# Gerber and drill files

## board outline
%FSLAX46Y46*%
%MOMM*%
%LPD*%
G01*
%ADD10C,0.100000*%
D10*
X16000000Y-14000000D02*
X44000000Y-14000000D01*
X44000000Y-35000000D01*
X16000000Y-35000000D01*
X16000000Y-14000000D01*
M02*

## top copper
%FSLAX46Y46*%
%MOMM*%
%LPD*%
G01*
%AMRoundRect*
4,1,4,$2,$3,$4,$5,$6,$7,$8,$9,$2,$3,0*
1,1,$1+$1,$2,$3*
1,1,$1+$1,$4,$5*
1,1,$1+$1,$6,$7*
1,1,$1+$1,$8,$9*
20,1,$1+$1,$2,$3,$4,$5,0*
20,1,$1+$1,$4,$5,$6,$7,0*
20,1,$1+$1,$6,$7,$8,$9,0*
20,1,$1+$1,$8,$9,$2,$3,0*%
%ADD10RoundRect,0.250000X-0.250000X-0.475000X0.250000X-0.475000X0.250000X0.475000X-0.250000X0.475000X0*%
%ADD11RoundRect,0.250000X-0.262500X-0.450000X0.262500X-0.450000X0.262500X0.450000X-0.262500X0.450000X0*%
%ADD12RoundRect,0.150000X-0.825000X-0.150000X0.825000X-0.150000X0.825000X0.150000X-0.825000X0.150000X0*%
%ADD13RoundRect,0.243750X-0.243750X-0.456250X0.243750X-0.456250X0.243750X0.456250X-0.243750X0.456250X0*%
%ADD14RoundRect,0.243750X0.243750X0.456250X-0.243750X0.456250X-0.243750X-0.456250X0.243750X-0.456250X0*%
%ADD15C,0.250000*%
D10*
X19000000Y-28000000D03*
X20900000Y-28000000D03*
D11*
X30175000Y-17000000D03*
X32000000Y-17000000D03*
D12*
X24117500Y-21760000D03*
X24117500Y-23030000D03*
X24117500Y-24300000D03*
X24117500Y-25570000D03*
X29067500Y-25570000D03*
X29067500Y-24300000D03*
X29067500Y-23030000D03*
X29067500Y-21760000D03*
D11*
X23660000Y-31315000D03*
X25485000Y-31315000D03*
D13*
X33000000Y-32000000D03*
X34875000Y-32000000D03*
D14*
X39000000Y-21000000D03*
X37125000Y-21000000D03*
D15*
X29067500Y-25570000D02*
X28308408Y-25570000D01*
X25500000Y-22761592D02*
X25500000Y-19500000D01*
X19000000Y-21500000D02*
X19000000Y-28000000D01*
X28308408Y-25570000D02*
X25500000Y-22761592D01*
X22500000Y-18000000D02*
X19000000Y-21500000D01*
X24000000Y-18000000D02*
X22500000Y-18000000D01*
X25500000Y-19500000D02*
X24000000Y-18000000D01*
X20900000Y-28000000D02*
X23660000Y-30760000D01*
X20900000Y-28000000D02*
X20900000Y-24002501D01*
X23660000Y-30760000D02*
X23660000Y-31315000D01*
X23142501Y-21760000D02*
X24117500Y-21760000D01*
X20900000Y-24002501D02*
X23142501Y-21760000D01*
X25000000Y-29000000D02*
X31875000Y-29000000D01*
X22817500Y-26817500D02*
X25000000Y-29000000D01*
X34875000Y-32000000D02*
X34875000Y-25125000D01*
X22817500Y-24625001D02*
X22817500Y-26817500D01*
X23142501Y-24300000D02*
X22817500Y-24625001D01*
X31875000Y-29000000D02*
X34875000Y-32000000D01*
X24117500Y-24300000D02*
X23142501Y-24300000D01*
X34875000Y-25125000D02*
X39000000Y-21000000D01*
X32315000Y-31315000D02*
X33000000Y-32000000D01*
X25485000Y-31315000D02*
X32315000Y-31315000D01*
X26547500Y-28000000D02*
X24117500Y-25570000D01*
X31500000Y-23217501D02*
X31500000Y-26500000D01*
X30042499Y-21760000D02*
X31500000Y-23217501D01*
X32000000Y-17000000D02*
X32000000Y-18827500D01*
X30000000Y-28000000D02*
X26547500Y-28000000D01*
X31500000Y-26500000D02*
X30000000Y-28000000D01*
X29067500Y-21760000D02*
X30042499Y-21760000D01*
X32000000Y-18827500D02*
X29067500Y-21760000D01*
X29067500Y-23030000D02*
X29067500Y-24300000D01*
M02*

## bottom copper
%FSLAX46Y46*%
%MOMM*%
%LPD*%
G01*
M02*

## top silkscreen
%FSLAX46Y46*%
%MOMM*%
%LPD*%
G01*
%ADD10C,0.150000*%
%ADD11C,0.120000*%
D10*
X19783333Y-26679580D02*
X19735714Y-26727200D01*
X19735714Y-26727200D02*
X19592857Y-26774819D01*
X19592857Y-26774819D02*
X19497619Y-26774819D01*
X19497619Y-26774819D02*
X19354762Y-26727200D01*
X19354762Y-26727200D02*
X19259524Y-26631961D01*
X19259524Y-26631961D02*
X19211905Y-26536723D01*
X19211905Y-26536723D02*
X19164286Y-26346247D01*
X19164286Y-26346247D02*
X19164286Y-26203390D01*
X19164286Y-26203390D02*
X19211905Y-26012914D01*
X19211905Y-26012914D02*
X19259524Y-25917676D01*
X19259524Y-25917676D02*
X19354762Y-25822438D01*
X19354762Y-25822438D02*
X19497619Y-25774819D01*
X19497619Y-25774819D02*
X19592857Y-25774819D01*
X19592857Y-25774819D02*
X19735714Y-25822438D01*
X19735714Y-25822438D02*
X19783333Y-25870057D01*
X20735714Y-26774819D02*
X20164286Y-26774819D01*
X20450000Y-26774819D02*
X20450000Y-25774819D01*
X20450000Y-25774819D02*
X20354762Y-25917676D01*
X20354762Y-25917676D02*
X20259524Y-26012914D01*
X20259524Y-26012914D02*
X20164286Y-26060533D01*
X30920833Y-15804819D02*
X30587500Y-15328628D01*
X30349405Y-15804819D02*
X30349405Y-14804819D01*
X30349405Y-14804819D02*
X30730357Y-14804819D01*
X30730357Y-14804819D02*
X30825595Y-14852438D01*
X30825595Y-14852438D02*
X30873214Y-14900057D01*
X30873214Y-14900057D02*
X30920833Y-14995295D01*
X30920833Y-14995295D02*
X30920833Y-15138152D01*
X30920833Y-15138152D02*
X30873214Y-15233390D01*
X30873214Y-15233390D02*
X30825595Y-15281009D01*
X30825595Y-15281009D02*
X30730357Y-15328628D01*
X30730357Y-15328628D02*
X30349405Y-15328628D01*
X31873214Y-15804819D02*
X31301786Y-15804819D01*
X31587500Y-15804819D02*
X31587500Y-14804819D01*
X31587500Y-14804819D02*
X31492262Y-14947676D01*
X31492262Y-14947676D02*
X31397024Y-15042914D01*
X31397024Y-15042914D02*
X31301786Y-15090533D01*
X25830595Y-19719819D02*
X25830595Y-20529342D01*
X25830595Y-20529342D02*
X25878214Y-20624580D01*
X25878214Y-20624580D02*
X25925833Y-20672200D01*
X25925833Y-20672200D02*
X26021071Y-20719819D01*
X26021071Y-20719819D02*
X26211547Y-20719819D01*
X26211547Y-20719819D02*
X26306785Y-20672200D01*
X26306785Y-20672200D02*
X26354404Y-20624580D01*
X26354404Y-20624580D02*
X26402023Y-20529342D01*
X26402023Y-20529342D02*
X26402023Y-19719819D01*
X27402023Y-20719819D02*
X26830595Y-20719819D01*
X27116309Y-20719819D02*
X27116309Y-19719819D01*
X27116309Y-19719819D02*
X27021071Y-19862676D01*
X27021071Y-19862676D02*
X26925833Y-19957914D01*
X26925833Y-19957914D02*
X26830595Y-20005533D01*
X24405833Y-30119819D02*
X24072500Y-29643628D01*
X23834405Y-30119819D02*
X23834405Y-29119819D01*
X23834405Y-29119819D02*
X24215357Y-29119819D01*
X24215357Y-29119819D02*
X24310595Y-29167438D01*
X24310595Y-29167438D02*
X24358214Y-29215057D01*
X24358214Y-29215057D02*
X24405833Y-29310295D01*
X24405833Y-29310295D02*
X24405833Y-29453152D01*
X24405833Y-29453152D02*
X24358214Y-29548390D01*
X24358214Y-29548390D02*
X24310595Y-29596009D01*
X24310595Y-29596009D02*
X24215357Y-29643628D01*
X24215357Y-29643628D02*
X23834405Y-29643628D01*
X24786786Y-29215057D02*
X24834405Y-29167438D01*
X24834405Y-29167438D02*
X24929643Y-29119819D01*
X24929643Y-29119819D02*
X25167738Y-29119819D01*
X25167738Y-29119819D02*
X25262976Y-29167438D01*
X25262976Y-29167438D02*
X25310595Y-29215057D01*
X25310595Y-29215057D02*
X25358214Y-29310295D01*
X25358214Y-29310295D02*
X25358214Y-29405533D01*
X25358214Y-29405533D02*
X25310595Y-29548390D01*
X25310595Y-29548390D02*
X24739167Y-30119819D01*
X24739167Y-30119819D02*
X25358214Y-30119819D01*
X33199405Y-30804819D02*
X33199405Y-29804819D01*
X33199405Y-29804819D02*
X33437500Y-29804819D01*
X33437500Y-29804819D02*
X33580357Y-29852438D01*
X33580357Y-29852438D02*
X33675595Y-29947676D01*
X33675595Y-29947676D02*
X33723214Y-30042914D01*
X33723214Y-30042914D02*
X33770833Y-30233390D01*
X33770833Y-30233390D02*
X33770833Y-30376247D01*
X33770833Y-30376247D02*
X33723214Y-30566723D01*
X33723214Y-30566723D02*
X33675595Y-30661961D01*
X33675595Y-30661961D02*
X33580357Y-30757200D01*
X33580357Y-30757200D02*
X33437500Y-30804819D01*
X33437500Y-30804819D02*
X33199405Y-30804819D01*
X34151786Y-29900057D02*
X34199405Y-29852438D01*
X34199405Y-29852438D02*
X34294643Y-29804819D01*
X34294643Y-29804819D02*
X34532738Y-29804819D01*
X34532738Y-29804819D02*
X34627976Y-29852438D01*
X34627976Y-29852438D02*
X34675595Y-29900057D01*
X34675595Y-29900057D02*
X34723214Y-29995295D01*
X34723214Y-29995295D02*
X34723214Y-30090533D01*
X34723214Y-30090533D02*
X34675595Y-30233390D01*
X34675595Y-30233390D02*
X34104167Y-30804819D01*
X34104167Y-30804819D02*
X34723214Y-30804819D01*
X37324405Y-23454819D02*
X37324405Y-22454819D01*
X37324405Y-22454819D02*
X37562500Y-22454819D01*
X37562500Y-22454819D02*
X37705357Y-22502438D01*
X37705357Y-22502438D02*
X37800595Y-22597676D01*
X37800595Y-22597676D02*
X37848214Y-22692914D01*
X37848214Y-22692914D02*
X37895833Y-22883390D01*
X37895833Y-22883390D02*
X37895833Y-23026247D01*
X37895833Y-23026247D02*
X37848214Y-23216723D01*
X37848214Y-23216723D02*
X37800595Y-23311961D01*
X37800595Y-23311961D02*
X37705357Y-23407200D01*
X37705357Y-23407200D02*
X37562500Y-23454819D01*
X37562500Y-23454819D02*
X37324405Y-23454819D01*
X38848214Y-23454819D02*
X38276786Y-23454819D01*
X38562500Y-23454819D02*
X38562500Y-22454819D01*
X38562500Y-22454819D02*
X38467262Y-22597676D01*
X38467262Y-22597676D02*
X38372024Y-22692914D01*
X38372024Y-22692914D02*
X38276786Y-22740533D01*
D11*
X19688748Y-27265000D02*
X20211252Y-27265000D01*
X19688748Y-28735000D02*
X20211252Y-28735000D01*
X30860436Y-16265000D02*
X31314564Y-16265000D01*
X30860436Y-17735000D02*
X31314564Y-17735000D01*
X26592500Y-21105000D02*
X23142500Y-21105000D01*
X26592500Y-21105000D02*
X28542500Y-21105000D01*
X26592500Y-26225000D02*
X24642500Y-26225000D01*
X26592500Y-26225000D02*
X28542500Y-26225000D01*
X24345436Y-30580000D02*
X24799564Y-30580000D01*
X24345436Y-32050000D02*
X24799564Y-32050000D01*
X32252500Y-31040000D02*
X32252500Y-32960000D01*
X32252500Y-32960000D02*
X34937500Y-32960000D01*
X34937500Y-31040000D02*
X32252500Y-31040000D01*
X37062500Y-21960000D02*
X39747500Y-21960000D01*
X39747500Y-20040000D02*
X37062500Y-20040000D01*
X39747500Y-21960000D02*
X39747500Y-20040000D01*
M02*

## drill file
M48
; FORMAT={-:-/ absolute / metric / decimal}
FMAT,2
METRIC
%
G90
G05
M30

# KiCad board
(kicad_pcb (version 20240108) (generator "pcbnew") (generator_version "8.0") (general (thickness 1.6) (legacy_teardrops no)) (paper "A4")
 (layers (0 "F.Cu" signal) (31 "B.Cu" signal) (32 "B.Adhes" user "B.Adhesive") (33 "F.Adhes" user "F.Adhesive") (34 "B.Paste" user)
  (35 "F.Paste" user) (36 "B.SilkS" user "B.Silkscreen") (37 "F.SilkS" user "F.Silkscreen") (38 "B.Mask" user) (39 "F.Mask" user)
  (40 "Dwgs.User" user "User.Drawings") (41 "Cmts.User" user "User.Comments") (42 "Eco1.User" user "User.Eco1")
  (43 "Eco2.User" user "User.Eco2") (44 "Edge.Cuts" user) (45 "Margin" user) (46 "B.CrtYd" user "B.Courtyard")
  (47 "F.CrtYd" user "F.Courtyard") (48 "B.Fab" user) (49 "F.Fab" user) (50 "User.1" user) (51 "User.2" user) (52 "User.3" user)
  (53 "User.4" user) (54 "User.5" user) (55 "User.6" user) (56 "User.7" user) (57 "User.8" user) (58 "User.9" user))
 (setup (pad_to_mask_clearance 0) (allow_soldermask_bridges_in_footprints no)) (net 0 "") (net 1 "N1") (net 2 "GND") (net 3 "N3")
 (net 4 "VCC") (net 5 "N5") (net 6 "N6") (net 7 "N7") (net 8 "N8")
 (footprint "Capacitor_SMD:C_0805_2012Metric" (layer "F.Cu") (at 19.95 28)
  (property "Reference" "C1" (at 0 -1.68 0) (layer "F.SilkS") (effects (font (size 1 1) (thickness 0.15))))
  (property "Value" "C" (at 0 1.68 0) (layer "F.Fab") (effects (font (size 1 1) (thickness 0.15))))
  (fp_line (start -0.261252 -0.735) (end 0.261252 -0.735) (stroke (width 0.12) (type solid)) (layer "F.SilkS"))
  (fp_line (start -0.261252 0.735) (end 0.261252 0.735) (stroke (width 0.12) (type solid)) (layer "F.SilkS"))
  (pad "1" smd roundrect (at -0.95 0) (size 1 1.45) (layers "F.Cu" "F.Paste" "F.Mask") (roundrect_rratio 0.25) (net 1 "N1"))
  (pad "2" smd roundrect (at 0.95 0) (size 1 1.45) (layers "F.Cu" "F.Paste" "F.Mask") (roundrect_rratio 0.25) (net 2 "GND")))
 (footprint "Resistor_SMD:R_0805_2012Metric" (layer "F.Cu") (at 31.0875 17)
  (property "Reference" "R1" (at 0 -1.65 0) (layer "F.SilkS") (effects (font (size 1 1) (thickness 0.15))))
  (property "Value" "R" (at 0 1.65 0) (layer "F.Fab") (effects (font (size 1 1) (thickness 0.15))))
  (fp_line (start -0.227064 -0.735) (end 0.227064 -0.735) (stroke (width 0.12) (type solid)) (layer "F.SilkS"))
  (fp_line (start -0.227064 0.735) (end 0.227064 0.735) (stroke (width 0.12) (type solid)) (layer "F.SilkS"))
  (pad "1" smd roundrect (at -0.9125 0) (size 1.025 1.4) (layers "F.Cu" "F.Paste" "F.Mask") (roundrect_rratio 0.243902) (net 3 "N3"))
  (pad "2" smd roundrect (at 0.9125 0) (size 1.025 1.4) (layers "F.Cu" "F.Paste" "F.Mask") (roundrect_rratio 0.243902) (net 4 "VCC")))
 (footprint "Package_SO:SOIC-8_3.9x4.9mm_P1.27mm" (layer "F.Cu") (at 26.5925 23.665)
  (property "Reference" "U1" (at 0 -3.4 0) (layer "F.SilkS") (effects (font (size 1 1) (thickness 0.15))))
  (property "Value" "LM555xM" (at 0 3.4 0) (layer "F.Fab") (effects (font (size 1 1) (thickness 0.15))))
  (fp_line (start 0 -2.56) (end -3.45 -2.56) (stroke (width 0.12) (type solid)) (layer "F.SilkS"))
  (fp_line (start 0 -2.56) (end 1.95 -2.56) (stroke (width 0.12) (type solid)) (layer "F.SilkS"))
  (fp_line (start 0 2.56) (end -1.95 2.56) (stroke (width 0.12) (type solid)) (layer "F.SilkS"))
  (fp_line (start 0 2.56) (end 1.95 2.56) (stroke (width 0.12) (type solid)) (layer "F.SilkS"))
  (pad "1" smd roundrect (at -2.475 -1.905) (size 1.95 0.6) (layers "F.Cu" "F.Paste" "F.Mask") (roundrect_rratio 0.25) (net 2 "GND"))
  (pad "2" smd roundrect (at -2.475 -0.635) (size 1.95 0.6) (layers "F.Cu" "F.Paste" "F.Mask") (roundrect_rratio 0.25) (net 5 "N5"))
  (pad "3" smd roundrect (at -2.475 0.635) (size 1.95 0.6) (layers "F.Cu" "F.Paste" "F.Mask") (roundrect_rratio 0.25) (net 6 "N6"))
  (pad "4" smd roundrect (at -2.475 1.905) (size 1.95 0.6) (layers "F.Cu" "F.Paste" "F.Mask") (roundrect_rratio 0.25) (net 4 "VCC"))
  (pad "5" smd roundrect (at 2.475 1.905) (size 1.95 0.6) (layers "F.Cu" "F.Paste" "F.Mask") (roundrect_rratio 0.25) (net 1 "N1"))
  (pad "6" smd roundrect (at 2.475 0.635) (size 1.95 0.6) (layers "F.Cu" "F.Paste" "F.Mask") (roundrect_rratio 0.25) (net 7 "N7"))
  (pad "7" smd roundrect (at 2.475 -0.635) (size 1.95 0.6) (layers "F.Cu" "F.Paste" "F.Mask") (roundrect_rratio 0.25) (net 7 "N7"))
  (pad "8" smd roundrect (at 2.475 -1.905) (size 1.95 0.6) (layers "F.Cu" "F.Paste" "F.Mask") (roundrect_rratio 0.25) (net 4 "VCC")))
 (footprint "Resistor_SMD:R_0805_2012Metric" (layer "F.Cu") (at 24.5725 31.315)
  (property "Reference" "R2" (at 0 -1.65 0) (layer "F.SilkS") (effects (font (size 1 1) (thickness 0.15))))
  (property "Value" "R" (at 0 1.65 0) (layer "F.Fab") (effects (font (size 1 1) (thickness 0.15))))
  (fp_line (start -0.227064 -0.735) (end 0.227064 -0.735) (stroke (width 0.12) (type solid)) (layer "F.SilkS"))
  (fp_line (start -0.227064 0.735) (end 0.227064 0.735) (stroke (width 0.12) (type solid)) (layer "F.SilkS"))
  (pad "1" smd roundrect (at -0.9125 0) (size 1.025 1.4) (layers "F.Cu" "F.Paste" "F.Mask") (roundrect_rratio 0.243902) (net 2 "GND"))
  (pad "2" smd roundrect (at 0.9125 0) (size 1.025 1.4) (layers "F.Cu" "F.Paste" "F.Mask") (roundrect_rratio 0.243902) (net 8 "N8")))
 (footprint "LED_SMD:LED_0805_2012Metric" (layer "F.Cu") (at 33.9375 32)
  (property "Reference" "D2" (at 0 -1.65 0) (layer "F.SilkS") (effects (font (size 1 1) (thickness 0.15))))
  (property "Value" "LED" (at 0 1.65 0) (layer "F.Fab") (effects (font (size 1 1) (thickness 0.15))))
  (fp_line (start -1.685 -0.96) (end -1.685 0.96) (stroke (width 0.12) (type solid)) (layer "F.SilkS"))
  (fp_line (start -1.685 0.96) (end 1 0.96) (stroke (width 0.12) (type solid)) (layer "F.SilkS"))
  (fp_line (start 1 -0.96) (end -1.685 -0.96) (stroke (width 0.12) (type solid)) (layer "F.SilkS"))
  (pad "1" smd roundrect (at -0.9375 0) (size 0.975 1.4) (layers "F.Cu" "F.Paste" "F.Mask") (roundrect_rratio 0.25) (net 8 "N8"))
  (pad "2" smd roundrect (at 0.9375 0) (size 0.975 1.4) (layers "F.Cu" "F.Paste" "F.Mask") (roundrect_rratio 0.25) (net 6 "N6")))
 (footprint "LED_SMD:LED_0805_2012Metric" (layer "F.Cu") (at 38.0625 21 180)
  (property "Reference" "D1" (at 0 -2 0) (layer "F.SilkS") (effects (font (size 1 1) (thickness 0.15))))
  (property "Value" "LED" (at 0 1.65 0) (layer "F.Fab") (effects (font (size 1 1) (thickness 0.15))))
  (fp_line (start 1 -0.96) (end -1.685 -0.96) (stroke (width 0.12) (type solid)) (layer "F.SilkS"))
  (fp_line (start -1.685 0.96) (end 1 0.96) (stroke (width 0.12) (type solid)) (layer "F.SilkS"))
  (fp_line (start -1.685 -0.96) (end -1.685 0.96) (stroke (width 0.12) (type solid)) (layer "F.SilkS"))
  (pad "1" smd roundrect (at -0.9375 0 180) (size 0.975 1.4) (layers "F.Cu" "F.Paste" "F.Mask") (roundrect_rratio 0.25) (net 6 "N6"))
  (pad "2" smd roundrect (at 0.9375 0 180) (size 0.975 1.4) (layers "F.Cu" "F.Paste" "F.Mask") (roundrect_rratio 0.25) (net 3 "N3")))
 (gr_rect (start 16 14) (end 44 35) (stroke (width 0.1) (type default)) (fill none) (layer "Edge.Cuts"))
 (segment (start 29.0675 25.57) (end 28.308408 25.57) (width 0.25) (layer "F.Cu") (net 1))
 (segment (start 25.5 22.761592) (end 25.5 19.5) (width 0.25) (layer "F.Cu") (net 1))
 (segment (start 19 21.5) (end 19 28) (width 0.25) (layer "F.Cu") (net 1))
 (segment (start 28.308408 25.57) (end 25.5 22.761592) (width 0.25) (layer "F.Cu") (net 1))
 (segment (start 22.5 18) (end 19 21.5) (width 0.25) (layer "F.Cu") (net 1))
 (segment (start 24 18) (end 22.5 18) (width 0.25) (layer "F.Cu") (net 1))
 (segment (start 25.5 19.5) (end 24 18) (width 0.25) (layer "F.Cu") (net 1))
 (segment (start 20.9 28) (end 23.66 30.76) (width 0.25) (layer "F.Cu") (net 2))
 (segment (start 20.9 28) (end 20.9 24.002501) (width 0.25) (layer "F.Cu") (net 2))
 (segment (start 23.66 30.76) (end 23.66 31.315) (width 0.25) (layer "F.Cu") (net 2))
 (segment (start 23.142501 21.76) (end 24.1175 21.76) (width 0.25) (layer "F.Cu") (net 2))
 (segment (start 20.9 24.002501) (end 23.142501 21.76) (width 0.25) (layer "F.Cu") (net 2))
 (segment (start 25 29) (end 31.875 29) (width 0.25) (layer "F.Cu") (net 6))
 (segment (start 22.8175 26.8175) (end 25 29) (width 0.25) (layer "F.Cu") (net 6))
 (segment (start 34.875 32) (end 34.875 25.125) (width 0.25) (layer "F.Cu") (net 6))
 (segment (start 22.8175 24.625001) (end 22.8175 26.8175) (width 0.25) (layer "F.Cu") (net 6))
 (segment (start 23.142501 24.3) (end 22.8175 24.625001) (width 0.25) (layer "F.Cu") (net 6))
 (segment (start 31.875 29) (end 34.875 32) (width 0.25) (layer "F.Cu") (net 6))
 (segment (start 24.1175 24.3) (end 23.142501 24.3) (width 0.25) (layer "F.Cu") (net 6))
 (segment (start 34.875 25.125) (end 39 21) (width 0.25) (layer "F.Cu") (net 6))
 (segment (start 32.315 31.315) (end 33 32) (width 0.25) (layer "F.Cu") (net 8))
 (segment (start 25.485 31.315) (end 32.315 31.315) (width 0.25) (layer "F.Cu") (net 8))
 (segment (start 26.5475 28) (end 24.1175 25.57) (width 0.25) (layer "F.Cu") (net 4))
 (segment (start 31.5 23.217501) (end 31.5 26.5) (width 0.25) (layer "F.Cu") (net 4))
 (segment (start 30.042499 21.76) (end 31.5 23.217501) (width 0.25) (layer "F.Cu") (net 4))
 (segment (start 32 17) (end 32 18.8275) (width 0.25) (layer "F.Cu") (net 4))
 (segment (start 30 28) (end 26.5475 28) (width 0.25) (layer "F.Cu") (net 4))
 (segment (start 31.5 26.5) (end 30 28) (width 0.25) (layer "F.Cu") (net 4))
 (segment (start 29.0675 21.76) (end 30.042499 21.76) (width 0.25) (layer "F.Cu") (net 4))
 (segment (start 32 18.8275) (end 29.0675 21.76) (width 0.25) (layer "F.Cu") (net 4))
 (segment (start 29.0675 23.03) (end 29.0675 24.3) (width 0.25) (layer "F.Cu") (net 7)))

